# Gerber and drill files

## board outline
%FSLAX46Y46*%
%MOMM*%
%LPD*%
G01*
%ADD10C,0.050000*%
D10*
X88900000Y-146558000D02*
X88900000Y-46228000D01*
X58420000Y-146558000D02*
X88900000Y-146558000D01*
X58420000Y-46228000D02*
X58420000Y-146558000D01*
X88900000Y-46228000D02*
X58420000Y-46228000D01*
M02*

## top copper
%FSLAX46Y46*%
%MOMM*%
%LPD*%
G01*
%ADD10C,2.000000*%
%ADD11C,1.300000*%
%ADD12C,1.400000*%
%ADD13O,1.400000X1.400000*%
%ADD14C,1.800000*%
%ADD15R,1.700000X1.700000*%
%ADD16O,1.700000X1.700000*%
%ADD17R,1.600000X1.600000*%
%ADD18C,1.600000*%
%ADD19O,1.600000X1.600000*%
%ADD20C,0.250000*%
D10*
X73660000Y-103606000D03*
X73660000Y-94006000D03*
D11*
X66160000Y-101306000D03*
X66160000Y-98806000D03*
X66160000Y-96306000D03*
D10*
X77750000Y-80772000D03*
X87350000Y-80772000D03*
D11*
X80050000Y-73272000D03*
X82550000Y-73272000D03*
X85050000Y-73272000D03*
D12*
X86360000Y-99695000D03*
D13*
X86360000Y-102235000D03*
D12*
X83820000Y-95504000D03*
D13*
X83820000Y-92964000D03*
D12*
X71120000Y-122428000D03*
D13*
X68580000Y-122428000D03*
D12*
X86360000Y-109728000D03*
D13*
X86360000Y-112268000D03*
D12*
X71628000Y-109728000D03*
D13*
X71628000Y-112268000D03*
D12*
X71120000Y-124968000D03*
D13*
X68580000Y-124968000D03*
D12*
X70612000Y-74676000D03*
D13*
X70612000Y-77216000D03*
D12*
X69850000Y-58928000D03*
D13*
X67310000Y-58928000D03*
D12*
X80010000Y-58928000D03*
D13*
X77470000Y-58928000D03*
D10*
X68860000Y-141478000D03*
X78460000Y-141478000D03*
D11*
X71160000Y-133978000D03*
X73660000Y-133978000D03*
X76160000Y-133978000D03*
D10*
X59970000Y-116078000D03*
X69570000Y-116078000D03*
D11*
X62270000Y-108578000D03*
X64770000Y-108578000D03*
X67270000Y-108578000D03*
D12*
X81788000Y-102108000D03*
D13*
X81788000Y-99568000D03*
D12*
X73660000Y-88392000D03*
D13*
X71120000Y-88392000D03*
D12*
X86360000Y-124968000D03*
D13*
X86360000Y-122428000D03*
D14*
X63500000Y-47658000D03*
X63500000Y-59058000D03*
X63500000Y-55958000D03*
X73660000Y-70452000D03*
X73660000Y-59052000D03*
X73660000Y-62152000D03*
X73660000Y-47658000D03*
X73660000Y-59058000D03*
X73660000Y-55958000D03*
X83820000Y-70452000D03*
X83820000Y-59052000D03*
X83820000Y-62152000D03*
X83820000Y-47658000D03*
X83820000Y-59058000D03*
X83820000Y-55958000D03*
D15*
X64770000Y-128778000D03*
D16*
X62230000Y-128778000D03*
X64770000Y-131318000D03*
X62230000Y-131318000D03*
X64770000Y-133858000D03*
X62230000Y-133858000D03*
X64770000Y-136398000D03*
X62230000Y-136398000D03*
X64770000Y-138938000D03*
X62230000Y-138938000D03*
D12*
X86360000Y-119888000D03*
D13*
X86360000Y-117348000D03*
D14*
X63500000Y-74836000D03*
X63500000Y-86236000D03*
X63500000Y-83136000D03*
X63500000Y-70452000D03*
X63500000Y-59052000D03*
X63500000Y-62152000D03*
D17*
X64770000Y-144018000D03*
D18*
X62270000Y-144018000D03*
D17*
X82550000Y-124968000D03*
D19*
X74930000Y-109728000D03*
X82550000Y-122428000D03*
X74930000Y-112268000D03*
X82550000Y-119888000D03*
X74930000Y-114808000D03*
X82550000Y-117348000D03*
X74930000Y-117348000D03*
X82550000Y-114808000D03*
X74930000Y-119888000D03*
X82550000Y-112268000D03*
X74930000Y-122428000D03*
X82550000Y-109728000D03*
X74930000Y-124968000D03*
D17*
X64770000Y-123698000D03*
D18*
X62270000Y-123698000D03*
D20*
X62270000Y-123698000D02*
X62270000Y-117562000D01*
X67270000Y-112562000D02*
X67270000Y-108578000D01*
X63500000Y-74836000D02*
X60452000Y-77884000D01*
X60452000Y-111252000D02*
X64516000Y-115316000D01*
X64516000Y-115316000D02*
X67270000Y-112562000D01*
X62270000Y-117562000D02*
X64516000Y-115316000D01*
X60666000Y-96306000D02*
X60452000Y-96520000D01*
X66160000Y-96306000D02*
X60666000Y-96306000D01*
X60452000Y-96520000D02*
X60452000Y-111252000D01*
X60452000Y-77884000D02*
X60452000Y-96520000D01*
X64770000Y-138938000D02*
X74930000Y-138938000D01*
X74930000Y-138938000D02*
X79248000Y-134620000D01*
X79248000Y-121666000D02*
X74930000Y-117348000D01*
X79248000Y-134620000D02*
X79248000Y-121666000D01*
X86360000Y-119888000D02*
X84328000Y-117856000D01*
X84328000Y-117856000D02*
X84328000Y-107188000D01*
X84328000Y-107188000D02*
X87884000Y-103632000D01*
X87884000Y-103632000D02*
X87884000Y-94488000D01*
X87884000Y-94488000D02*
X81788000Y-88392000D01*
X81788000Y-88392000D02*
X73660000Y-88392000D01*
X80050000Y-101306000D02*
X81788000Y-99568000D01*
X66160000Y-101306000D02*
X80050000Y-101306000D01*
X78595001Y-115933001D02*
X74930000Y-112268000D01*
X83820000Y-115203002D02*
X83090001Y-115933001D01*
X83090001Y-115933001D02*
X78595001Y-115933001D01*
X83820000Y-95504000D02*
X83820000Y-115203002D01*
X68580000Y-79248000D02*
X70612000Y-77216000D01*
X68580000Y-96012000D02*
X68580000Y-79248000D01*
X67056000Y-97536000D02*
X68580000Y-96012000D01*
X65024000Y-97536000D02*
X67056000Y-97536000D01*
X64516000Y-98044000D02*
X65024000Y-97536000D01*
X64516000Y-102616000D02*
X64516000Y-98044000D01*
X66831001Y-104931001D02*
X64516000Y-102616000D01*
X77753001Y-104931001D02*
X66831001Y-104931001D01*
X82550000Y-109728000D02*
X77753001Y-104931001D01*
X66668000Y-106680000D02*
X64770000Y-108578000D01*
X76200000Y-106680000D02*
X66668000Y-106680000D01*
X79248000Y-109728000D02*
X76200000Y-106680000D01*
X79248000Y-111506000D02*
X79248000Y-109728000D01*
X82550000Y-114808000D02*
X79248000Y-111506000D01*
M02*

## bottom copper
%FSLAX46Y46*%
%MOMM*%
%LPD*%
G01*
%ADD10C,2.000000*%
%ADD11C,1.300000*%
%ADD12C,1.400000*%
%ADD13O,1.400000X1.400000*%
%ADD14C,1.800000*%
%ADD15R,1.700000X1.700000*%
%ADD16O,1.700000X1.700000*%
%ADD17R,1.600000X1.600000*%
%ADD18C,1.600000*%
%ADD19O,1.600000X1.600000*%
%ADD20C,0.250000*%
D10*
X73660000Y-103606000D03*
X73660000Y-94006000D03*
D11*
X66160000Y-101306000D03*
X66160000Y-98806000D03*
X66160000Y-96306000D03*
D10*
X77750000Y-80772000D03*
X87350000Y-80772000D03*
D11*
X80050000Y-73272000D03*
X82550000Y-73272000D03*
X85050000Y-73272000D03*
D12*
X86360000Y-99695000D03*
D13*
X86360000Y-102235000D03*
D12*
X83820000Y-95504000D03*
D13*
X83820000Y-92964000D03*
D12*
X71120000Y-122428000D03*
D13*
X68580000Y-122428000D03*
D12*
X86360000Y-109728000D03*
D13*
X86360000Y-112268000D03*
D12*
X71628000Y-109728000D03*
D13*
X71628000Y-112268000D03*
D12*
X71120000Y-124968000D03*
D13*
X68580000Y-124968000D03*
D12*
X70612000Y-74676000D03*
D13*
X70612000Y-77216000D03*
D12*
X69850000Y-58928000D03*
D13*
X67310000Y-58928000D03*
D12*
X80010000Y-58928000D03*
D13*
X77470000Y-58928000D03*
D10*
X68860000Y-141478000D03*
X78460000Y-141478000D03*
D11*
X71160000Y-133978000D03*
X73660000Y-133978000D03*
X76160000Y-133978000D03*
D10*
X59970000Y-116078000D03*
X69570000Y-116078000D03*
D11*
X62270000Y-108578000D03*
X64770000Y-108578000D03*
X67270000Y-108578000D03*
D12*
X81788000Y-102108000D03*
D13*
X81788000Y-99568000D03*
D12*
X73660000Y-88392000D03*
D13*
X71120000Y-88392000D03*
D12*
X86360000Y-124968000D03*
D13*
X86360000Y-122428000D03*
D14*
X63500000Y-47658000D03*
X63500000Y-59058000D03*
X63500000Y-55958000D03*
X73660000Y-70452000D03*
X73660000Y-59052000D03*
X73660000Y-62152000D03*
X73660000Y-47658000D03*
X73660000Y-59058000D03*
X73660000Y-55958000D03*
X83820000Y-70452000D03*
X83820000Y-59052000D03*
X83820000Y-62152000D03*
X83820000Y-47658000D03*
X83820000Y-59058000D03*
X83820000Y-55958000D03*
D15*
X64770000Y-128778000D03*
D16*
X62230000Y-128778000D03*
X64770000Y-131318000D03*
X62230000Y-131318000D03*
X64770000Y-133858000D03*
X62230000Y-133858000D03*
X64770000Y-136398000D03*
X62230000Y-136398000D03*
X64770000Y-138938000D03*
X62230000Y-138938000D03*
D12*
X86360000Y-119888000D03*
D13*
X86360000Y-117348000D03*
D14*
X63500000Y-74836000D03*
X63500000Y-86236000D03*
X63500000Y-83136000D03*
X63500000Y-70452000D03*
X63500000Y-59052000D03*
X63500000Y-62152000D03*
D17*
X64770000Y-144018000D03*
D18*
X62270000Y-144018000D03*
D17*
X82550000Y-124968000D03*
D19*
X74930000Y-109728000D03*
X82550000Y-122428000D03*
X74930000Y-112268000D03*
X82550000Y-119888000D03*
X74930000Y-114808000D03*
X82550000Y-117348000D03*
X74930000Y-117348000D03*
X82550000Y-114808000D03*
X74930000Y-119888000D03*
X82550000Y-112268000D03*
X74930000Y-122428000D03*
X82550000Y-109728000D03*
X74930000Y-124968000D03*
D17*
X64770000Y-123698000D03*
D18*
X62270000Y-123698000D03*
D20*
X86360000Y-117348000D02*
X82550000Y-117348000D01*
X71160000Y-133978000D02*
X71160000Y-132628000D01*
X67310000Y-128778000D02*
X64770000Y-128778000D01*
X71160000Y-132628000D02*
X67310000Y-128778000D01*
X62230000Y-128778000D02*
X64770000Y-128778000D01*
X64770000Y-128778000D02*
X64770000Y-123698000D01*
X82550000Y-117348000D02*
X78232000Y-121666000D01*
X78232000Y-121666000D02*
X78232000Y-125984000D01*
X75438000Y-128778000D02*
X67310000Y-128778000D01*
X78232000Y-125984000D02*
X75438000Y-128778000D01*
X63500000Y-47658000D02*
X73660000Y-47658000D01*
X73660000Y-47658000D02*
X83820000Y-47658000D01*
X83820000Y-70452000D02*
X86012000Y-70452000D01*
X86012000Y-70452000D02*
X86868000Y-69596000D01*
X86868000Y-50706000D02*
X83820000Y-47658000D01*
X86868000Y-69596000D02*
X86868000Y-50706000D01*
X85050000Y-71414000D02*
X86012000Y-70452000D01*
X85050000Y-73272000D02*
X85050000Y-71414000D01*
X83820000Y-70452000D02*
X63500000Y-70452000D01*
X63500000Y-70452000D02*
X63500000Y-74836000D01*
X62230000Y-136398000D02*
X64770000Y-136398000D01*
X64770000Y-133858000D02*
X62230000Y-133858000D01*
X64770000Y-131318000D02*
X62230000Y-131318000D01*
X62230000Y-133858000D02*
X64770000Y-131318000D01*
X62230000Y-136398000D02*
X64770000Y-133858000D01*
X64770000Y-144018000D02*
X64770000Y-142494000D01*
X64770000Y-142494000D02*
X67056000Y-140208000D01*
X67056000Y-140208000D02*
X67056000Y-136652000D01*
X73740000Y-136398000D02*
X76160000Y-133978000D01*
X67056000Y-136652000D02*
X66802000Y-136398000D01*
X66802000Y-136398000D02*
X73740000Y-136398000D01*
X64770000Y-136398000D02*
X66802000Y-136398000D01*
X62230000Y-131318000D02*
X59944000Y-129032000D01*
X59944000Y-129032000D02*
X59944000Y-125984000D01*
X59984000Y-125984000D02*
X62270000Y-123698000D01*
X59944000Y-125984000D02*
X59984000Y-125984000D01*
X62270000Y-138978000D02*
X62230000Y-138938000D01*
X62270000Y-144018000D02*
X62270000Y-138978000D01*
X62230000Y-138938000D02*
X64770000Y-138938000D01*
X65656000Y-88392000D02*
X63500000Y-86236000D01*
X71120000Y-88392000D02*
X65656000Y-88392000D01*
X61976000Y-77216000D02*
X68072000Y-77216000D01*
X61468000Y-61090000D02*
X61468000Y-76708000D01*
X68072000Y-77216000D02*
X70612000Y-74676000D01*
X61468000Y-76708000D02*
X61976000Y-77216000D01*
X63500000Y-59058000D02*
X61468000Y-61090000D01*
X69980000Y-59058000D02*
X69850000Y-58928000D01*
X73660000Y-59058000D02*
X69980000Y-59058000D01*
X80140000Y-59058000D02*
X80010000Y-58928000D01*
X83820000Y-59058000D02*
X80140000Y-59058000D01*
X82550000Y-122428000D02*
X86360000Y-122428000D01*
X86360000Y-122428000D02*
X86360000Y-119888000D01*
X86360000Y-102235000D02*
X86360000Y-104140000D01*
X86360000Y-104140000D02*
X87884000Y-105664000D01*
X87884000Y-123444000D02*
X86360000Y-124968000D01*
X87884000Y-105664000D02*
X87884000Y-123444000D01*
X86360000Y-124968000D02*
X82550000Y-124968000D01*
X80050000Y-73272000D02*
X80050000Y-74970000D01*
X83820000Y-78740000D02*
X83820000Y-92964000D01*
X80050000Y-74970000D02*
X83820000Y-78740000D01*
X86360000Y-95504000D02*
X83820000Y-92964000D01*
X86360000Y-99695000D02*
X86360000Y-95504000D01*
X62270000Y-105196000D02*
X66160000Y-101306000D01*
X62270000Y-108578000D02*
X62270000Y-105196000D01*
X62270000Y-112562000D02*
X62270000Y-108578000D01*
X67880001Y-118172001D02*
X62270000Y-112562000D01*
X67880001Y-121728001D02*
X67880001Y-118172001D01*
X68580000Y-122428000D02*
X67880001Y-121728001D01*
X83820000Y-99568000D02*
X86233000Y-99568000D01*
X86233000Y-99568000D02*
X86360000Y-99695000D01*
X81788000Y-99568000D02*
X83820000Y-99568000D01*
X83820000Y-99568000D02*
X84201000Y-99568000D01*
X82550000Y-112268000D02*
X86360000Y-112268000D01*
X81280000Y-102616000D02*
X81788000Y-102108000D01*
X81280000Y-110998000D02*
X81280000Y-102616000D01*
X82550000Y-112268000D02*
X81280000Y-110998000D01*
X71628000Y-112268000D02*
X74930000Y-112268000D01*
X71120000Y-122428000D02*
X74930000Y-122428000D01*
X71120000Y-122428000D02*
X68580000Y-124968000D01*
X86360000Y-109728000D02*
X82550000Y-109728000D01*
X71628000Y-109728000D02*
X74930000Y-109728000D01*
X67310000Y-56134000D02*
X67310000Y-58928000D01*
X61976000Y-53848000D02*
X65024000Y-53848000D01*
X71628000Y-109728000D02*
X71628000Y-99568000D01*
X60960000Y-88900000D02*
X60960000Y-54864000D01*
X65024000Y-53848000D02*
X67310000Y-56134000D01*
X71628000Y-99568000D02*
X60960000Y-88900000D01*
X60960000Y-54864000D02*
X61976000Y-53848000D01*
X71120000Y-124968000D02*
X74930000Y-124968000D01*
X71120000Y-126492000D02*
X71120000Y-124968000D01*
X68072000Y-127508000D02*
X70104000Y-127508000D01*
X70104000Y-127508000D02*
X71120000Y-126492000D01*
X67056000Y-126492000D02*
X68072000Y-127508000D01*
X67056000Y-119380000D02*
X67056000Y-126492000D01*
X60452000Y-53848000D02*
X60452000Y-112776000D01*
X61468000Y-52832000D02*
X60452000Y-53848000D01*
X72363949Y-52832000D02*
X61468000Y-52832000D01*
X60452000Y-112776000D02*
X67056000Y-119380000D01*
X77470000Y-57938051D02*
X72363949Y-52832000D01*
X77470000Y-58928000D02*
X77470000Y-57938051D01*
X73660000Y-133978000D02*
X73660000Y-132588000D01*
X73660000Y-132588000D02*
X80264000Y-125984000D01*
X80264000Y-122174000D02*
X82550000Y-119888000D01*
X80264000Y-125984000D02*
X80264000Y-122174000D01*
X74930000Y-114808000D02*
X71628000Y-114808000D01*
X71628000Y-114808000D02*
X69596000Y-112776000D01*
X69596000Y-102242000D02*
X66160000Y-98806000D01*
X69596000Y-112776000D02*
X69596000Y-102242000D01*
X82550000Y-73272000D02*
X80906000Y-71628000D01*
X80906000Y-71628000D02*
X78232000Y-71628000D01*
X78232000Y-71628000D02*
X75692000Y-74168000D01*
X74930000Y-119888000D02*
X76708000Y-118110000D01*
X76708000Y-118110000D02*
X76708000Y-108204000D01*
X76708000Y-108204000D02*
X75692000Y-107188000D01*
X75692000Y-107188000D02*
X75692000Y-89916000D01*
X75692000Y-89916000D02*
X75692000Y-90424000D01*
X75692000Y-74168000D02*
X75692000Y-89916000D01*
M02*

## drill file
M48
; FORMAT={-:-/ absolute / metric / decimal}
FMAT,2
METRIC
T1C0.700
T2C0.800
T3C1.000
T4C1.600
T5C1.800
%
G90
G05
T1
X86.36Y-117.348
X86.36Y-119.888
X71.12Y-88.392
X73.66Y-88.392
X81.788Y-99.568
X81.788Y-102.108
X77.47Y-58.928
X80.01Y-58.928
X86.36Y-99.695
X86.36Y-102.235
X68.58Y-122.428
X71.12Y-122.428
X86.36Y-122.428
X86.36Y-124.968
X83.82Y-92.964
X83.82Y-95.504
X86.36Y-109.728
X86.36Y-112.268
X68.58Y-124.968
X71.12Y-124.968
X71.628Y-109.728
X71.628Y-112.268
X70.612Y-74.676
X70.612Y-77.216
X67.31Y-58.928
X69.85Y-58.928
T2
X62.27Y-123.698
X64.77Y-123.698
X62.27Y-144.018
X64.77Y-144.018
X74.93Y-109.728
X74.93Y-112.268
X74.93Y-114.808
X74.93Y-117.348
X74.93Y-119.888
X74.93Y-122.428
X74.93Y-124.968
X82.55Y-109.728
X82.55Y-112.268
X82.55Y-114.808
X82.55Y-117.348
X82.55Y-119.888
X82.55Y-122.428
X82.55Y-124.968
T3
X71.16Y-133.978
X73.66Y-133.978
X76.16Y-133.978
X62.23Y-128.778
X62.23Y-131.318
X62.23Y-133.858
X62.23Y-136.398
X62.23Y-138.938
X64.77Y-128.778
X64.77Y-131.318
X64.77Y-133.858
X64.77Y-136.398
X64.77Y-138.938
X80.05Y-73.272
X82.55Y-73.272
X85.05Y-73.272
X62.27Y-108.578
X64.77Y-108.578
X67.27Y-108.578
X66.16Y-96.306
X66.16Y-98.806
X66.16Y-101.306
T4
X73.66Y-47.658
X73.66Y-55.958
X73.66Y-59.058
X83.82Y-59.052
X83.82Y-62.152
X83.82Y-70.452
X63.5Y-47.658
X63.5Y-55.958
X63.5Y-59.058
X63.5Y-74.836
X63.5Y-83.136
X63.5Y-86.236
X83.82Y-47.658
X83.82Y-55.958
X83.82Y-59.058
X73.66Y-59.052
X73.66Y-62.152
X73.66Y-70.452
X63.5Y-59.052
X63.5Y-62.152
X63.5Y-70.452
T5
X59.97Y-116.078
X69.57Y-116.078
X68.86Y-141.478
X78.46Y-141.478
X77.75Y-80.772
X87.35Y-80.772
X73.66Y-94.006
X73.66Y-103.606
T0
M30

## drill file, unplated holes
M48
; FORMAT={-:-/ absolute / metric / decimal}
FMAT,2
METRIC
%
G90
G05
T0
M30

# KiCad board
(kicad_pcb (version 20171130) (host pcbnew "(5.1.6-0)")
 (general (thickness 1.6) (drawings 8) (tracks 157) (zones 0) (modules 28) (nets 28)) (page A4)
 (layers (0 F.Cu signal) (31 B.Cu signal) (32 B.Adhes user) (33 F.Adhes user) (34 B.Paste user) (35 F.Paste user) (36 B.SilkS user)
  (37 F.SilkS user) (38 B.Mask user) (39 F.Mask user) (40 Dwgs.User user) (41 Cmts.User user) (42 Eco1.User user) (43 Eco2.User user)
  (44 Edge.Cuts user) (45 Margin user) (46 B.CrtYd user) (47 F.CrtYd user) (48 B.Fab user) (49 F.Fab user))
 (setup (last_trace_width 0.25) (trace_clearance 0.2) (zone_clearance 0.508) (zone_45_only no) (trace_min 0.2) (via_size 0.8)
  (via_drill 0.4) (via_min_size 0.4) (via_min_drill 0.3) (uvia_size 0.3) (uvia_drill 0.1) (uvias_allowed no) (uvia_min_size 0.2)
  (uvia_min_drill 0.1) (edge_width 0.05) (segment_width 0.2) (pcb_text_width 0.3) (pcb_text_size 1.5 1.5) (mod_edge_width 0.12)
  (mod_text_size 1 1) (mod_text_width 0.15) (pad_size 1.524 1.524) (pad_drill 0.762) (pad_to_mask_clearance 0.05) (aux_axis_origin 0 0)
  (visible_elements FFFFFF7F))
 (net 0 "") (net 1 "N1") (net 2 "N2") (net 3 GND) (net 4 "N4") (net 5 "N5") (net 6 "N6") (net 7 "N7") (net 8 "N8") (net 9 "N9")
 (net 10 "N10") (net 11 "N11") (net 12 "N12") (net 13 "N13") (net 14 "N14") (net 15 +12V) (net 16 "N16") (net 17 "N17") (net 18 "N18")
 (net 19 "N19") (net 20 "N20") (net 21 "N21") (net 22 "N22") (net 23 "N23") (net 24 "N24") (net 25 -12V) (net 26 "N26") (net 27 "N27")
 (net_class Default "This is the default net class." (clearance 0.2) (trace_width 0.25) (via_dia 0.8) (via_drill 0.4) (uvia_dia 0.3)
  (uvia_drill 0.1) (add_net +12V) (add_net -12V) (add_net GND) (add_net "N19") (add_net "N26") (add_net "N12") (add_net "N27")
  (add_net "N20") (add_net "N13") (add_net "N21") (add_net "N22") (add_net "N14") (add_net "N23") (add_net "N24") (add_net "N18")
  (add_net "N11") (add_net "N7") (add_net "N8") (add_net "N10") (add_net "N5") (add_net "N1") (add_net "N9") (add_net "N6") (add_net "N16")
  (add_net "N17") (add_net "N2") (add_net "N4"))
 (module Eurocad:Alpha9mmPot (layer F.Cu) (at 73.66 98.806 270)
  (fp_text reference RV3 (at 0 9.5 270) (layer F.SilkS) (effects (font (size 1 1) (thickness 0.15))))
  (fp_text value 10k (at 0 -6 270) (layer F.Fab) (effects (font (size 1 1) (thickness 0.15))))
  (pad "" thru_hole circle (at 4.8 0 270) (size 2 2) (drill 1.8) (layers *.Cu *.Mask F.SilkS))
  (pad "" thru_hole circle (at -4.8 0 270) (size 2 2) (drill 1.8) (layers *.Cu *.Mask F.SilkS))
  (pad 3 thru_hole circle (at 2.5 7.5 270) (size 1.3 1.3) (drill 1) (layers *.Cu *.Mask F.SilkS) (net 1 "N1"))
  (pad 2 thru_hole circle (at 0 7.5 270) (size 1.3 1.3) (drill 1) (layers *.Cu *.Mask F.SilkS) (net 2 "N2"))
  (pad 1 thru_hole circle (at -2.5 7.5 270) (size 1.3 1.3) (drill 1) (layers *.Cu *.Mask F.SilkS) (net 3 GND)))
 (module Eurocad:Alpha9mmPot (layer F.Cu) (at 82.55 80.772 180)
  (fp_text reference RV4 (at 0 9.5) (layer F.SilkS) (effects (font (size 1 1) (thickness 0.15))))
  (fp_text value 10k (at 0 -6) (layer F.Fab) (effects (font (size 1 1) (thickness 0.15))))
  (pad "" thru_hole circle (at 4.8 0 180) (size 2 2) (drill 1.8) (layers *.Cu *.Mask F.SilkS))
  (pad "" thru_hole circle (at -4.8 0 180) (size 2 2) (drill 1.8) (layers *.Cu *.Mask F.SilkS))
  (pad 3 thru_hole circle (at 2.5 7.5 180) (size 1.3 1.3) (drill 1) (layers *.Cu *.Mask F.SilkS) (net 1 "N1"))
  (pad 2 thru_hole circle (at 0 7.5 180) (size 1.3 1.3) (drill 1) (layers *.Cu *.Mask F.SilkS) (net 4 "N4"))
  (pad 1 thru_hole circle (at -2.5 7.5 180) (size 1.3 1.3) (drill 1) (layers *.Cu *.Mask F.SilkS) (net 3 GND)))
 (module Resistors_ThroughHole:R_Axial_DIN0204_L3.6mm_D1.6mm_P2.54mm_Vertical (layer F.Cu) (at 86.36 99.695 270)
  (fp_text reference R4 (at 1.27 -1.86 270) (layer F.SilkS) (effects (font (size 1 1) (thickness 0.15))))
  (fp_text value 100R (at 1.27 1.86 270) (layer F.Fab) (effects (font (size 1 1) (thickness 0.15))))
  (pad 1 thru_hole circle (at 0 0 270) (size 1.4 1.4) (drill 0.7) (layers *.Cu *.Mask) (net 1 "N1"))
  (pad 2 thru_hole oval (at 2.54 0 270) (size 1.4 1.4) (drill 0.7) (layers *.Cu *.Mask) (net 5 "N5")))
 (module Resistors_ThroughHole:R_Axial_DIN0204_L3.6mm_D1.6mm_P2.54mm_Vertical (layer F.Cu) (at 83.82 95.504 90)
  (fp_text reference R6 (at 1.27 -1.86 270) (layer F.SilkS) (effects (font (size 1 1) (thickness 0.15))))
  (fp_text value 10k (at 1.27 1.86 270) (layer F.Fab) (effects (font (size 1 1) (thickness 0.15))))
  (pad 1 thru_hole circle (at 0 0 90) (size 1.4 1.4) (drill 0.7) (layers *.Cu *.Mask) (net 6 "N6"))
  (pad 2 thru_hole oval (at 2.54 0 90) (size 1.4 1.4) (drill 0.7) (layers *.Cu *.Mask) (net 1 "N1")))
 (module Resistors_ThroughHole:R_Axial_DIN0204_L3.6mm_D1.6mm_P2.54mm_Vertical (layer F.Cu) (at 71.12 122.428 180)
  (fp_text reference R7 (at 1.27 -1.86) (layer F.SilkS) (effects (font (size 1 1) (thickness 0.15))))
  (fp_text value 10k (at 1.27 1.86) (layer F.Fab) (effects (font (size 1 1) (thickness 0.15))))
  (pad 1 thru_hole circle (at 0 0 180) (size 1.4 1.4) (drill 0.7) (layers *.Cu *.Mask) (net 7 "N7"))
  (pad 2 thru_hole oval (at 2.54 0 180) (size 1.4 1.4) (drill 0.7) (layers *.Cu *.Mask) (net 1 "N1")))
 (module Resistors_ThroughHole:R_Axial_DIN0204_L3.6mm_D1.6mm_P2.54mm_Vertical (layer F.Cu) (at 86.36 109.728 270)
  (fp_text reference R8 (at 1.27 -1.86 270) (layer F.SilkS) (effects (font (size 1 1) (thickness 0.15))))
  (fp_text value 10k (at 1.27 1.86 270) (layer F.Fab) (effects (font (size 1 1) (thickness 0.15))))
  (pad 1 thru_hole circle (at 0 0 270) (size 1.4 1.4) (drill 0.7) (layers *.Cu *.Mask) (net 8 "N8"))
  (pad 2 thru_hole oval (at 2.54 0 270) (size 1.4 1.4) (drill 0.7) (layers *.Cu *.Mask) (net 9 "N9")))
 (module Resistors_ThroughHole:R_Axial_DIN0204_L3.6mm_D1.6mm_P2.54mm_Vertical (layer F.Cu) (at 71.628 109.728 270)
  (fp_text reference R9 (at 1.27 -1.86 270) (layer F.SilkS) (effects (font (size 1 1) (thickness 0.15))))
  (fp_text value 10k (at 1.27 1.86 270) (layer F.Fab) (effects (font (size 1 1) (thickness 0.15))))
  (pad 1 thru_hole circle (at 0 0 270) (size 1.4 1.4) (drill 0.7) (layers *.Cu *.Mask) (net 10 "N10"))
  (pad 2 thru_hole oval (at 2.54 0 270) (size 1.4 1.4) (drill 0.7) (layers *.Cu *.Mask) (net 6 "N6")))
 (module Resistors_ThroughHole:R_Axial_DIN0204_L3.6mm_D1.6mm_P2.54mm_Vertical (layer F.Cu) (at 71.12 124.968 180)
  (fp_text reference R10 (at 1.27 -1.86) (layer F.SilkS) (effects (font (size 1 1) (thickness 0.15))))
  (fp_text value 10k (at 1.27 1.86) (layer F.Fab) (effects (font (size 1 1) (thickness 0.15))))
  (pad 1 thru_hole circle (at 0 0 180) (size 1.4 1.4) (drill 0.7) (layers *.Cu *.Mask) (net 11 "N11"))
  (pad 2 thru_hole oval (at 2.54 0 180) (size 1.4 1.4) (drill 0.7) (layers *.Cu *.Mask) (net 7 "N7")))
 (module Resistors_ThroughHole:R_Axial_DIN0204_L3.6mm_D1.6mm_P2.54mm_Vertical (layer F.Cu) (at 70.612 74.676 270)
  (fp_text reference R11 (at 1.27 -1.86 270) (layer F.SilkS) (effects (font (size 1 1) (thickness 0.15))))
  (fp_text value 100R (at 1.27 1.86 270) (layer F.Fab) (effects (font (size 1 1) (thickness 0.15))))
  (pad 1 thru_hole circle (at 0 0 270) (size 1.4 1.4) (drill 0.7) (layers *.Cu *.Mask) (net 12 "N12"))
  (pad 2 thru_hole oval (at 2.54 0 270) (size 1.4 1.4) (drill 0.7) (layers *.Cu *.Mask) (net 8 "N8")))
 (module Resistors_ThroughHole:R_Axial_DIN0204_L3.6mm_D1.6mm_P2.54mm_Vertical (layer F.Cu) (at 69.85 58.928 180)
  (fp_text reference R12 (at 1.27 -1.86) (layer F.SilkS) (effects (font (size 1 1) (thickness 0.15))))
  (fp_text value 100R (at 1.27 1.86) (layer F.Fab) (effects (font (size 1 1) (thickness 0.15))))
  (pad 1 thru_hole circle (at 0 0 180) (size 1.4 1.4) (drill 0.7) (layers *.Cu *.Mask) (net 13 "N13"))
  (pad 2 thru_hole oval (at 2.54 0 180) (size 1.4 1.4) (drill 0.7) (layers *.Cu *.Mask) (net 10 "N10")))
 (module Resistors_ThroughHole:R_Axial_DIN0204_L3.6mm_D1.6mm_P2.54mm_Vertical (layer F.Cu) (at 80.01 58.928 180)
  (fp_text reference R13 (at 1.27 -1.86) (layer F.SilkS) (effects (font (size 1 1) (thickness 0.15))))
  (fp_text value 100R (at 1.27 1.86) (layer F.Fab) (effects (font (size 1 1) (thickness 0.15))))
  (pad 1 thru_hole circle (at 0 0 180) (size 1.4 1.4) (drill 0.7) (layers *.Cu *.Mask) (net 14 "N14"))
  (pad 2 thru_hole oval (at 2.54 0 180) (size 1.4 1.4) (drill 0.7) (layers *.Cu *.Mask) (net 11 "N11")))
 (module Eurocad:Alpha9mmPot (layer F.Cu) (at 73.66 141.478 180)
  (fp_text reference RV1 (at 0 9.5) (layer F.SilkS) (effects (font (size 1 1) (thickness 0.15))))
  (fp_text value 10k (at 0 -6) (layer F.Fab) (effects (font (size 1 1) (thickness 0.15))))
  (pad "" thru_hole circle (at 4.8 0 180) (size 2 2) (drill 1.8) (layers *.Cu *.Mask F.SilkS))
  (pad "" thru_hole circle (at -4.8 0 180) (size 2 2) (drill 1.8) (layers *.Cu *.Mask F.SilkS))
  (pad 3 thru_hole circle (at 2.5 7.5 180) (size 1.3 1.3) (drill 1) (layers *.Cu *.Mask F.SilkS) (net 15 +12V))
  (pad 2 thru_hole circle (at 0 7.5 180) (size 1.3 1.3) (drill 1) (layers *.Cu *.Mask F.SilkS) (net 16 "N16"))
  (pad 1 thru_hole circle (at -2.5 7.5 180) (size 1.3 1.3) (drill 1) (layers *.Cu *.Mask F.SilkS) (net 3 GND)))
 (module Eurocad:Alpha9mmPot (layer F.Cu) (at 64.77 116.078 180)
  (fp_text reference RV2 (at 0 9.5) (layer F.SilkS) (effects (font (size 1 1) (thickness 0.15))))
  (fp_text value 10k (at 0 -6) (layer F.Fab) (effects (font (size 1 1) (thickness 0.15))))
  (pad "" thru_hole circle (at 4.8 0 180) (size 2 2) (drill 1.8) (layers *.Cu *.Mask F.SilkS))
  (pad "" thru_hole circle (at -4.8 0 180) (size 2 2) (drill 1.8) (layers *.Cu *.Mask F.SilkS))
  (pad 3 thru_hole circle (at 2.5 7.5 180) (size 1.3 1.3) (drill 1) (layers *.Cu *.Mask F.SilkS) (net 1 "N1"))
  (pad 2 thru_hole circle (at 0 7.5 180) (size 1.3 1.3) (drill 1) (layers *.Cu *.Mask F.SilkS) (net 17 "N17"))
  (pad 1 thru_hole circle (at -2.5 7.5 180) (size 1.3 1.3) (drill 1) (layers *.Cu *.Mask F.SilkS) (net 3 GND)))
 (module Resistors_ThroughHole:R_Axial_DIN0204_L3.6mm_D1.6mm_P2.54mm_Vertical (layer F.Cu) (at 81.788 102.108 90)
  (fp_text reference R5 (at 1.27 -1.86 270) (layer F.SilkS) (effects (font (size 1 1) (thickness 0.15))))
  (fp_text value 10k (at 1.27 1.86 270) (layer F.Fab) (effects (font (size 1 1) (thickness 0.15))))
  (pad 1 thru_hole circle (at 0 0 90) (size 1.4 1.4) (drill 0.7) (layers *.Cu *.Mask) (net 9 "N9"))
  (pad 2 thru_hole oval (at 2.54 0 90) (size 1.4 1.4) (drill 0.7) (layers *.Cu *.Mask) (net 1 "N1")))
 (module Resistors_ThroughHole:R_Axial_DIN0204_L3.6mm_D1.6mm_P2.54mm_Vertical (layer F.Cu) (at 73.66 88.392 180)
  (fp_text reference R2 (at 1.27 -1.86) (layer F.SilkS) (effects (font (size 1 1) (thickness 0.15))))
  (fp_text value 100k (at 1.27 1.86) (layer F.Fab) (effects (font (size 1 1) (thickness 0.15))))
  (pad 1 thru_hole circle (at 0 0 180) (size 1.4 1.4) (drill 0.7) (layers *.Cu *.Mask) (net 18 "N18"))
  (pad 2 thru_hole oval (at 2.54 0 180) (size 1.4 1.4) (drill 0.7) (layers *.Cu *.Mask) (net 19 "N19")))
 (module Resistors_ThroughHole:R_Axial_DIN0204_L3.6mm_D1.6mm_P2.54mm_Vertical (layer F.Cu) (at 86.36 124.968 90)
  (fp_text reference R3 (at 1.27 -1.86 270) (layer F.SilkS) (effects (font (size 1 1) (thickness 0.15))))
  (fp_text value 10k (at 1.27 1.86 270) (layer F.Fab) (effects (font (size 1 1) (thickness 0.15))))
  (pad 1 thru_hole circle (at 0 0 90) (size 1.4 1.4) (drill 0.7) (layers *.Cu *.Mask) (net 5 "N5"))
  (pad 2 thru_hole oval (at 2.54 0 90) (size 1.4 1.4) (drill 0.7) (layers *.Cu *.Mask) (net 18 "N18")))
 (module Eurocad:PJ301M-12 (layer F.Cu) (at 63.5 52.578)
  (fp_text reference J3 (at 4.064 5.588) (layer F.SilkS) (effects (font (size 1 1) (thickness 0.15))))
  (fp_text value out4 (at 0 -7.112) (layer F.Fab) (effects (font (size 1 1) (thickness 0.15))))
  (pad 3 thru_hole circle (at 0 -4.92) (size 1.8 1.8) (drill 1.6) (layers *.Cu *.Mask F.SilkS) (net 3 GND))
  (pad 1 thru_hole circle (at 0 6.48) (size 1.8 1.8) (drill 1.6) (layers *.Cu *.Mask F.SilkS) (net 12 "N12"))
  (pad 2 thru_hole circle (at 0 3.38) (size 1.8 1.8) (drill 1.6) (layers *.Cu *.Mask F.SilkS) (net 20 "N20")))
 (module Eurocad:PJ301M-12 (layer F.Cu) (at 73.66 65.532 180)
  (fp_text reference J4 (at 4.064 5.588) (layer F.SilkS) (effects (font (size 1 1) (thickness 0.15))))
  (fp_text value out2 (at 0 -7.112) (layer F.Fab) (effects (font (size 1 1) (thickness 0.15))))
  (pad 3 thru_hole circle (at 0 -4.92 180) (size 1.8 1.8) (drill 1.6) (layers *.Cu *.Mask F.SilkS) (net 3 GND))
  (pad 1 thru_hole circle (at 0 6.48 180) (size 1.8 1.8) (drill 1.6) (layers *.Cu *.Mask F.SilkS) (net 13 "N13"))
  (pad 2 thru_hole circle (at 0 3.38 180) (size 1.8 1.8) (drill 1.6) (layers *.Cu *.Mask F.SilkS) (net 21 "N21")))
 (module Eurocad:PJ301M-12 (layer F.Cu) (at 73.66 52.578)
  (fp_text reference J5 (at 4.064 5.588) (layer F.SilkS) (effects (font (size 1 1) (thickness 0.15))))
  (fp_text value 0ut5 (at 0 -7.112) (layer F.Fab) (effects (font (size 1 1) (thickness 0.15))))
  (pad 3 thru_hole circle (at 0 -4.92) (size 1.8 1.8) (drill 1.6) (layers *.Cu *.Mask F.SilkS) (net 3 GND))
  (pad 1 thru_hole circle (at 0 6.48) (size 1.8 1.8) (drill 1.6) (layers *.Cu *.Mask F.SilkS) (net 13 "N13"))
  (pad 2 thru_hole circle (at 0 3.38) (size 1.8 1.8) (drill 1.6) (layers *.Cu *.Mask F.SilkS) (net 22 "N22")))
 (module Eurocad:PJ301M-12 (layer F.Cu) (at 83.82 65.532 180)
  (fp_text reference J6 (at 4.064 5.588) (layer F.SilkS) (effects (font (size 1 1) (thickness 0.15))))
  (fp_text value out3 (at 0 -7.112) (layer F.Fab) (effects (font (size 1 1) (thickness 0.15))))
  (pad 3 thru_hole circle (at 0 -4.92 180) (size 1.8 1.8) (drill 1.6) (layers *.Cu *.Mask F.SilkS) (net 3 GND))
  (pad 1 thru_hole circle (at 0 6.48 180) (size 1.8 1.8) (drill 1.6) (layers *.Cu *.Mask F.SilkS) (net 14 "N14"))
  (pad 2 thru_hole circle (at 0 3.38 180) (size 1.8 1.8) (drill 1.6) (layers *.Cu *.Mask F.SilkS) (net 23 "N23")))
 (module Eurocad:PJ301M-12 (layer F.Cu) (at 83.82 52.578)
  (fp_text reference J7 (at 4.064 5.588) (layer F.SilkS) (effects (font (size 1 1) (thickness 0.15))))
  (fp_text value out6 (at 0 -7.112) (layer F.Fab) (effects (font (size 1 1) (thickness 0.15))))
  (pad 3 thru_hole circle (at 0 -4.92) (size 1.8 1.8) (drill 1.6) (layers *.Cu *.Mask F.SilkS) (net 3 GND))
  (pad 1 thru_hole circle (at 0 6.48) (size 1.8 1.8) (drill 1.6) (layers *.Cu *.Mask F.SilkS) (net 14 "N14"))
  (pad 2 thru_hole circle (at 0 3.38) (size 1.8 1.8) (drill 1.6) (layers *.Cu *.Mask F.SilkS) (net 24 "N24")))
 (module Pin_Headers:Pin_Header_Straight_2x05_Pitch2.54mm (layer B.Cu) (at 64.77 128.778 180)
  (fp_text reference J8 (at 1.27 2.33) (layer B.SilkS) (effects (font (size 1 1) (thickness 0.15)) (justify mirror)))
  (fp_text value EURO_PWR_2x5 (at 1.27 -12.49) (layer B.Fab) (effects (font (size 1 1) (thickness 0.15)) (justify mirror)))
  (pad 1 thru_hole rect (at 0 0 180) (size 1.7 1.7) (drill 1) (layers *.Cu *.Mask) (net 15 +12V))
  (pad 2 thru_hole oval (at 2.54 0 180) (size 1.7 1.7) (drill 1) (layers *.Cu *.Mask) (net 15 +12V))
  (pad 3 thru_hole oval (at 0 -2.54 180) (size 1.7 1.7) (drill 1) (layers *.Cu *.Mask) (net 3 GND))
  (pad 4 thru_hole oval (at 2.54 -2.54 180) (size 1.7 1.7) (drill 1) (layers *.Cu *.Mask) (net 3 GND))
  (pad 5 thru_hole oval (at 0 -5.08 180) (size 1.7 1.7) (drill 1) (layers *.Cu *.Mask) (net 3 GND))
  (pad 6 thru_hole oval (at 2.54 -5.08 180) (size 1.7 1.7) (drill 1) (layers *.Cu *.Mask) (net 3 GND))
  (pad 7 thru_hole oval (at 0 -7.62 180) (size 1.7 1.7) (drill 1) (layers *.Cu *.Mask) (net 3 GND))
  (pad 8 thru_hole oval (at 2.54 -7.62 180) (size 1.7 1.7) (drill 1) (layers *.Cu *.Mask) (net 3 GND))
  (pad 9 thru_hole oval (at 0 -10.16 180) (size 1.7 1.7) (drill 1) (layers *.Cu *.Mask) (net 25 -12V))
  (pad 10 thru_hole oval (at 2.54 -10.16 180) (size 1.7 1.7) (drill 1) (layers *.Cu *.Mask) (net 25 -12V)))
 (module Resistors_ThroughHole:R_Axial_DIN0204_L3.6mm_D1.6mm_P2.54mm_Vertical (layer F.Cu) (at 86.36 119.888 90)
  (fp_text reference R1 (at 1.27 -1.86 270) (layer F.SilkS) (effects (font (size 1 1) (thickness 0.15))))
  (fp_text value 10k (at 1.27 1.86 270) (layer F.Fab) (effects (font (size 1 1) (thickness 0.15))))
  (pad 1 thru_hole circle (at 0 0 90) (size 1.4 1.4) (drill 0.7) (layers *.Cu *.Mask) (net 18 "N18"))
  (pad 2 thru_hole oval (at 2.54 0 90) (size 1.4 1.4) (drill 0.7) (layers *.Cu *.Mask) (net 15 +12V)))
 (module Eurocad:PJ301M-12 (layer F.Cu) (at 63.5 79.756)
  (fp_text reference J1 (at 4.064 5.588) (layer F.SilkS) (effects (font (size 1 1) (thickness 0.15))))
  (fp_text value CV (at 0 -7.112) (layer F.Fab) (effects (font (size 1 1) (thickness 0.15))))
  (pad 3 thru_hole circle (at 0 -4.92) (size 1.8 1.8) (drill 1.6) (layers *.Cu *.Mask F.SilkS) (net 3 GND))
  (pad 1 thru_hole circle (at 0 6.48) (size 1.8 1.8) (drill 1.6) (layers *.Cu *.Mask F.SilkS) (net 19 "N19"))
  (pad 2 thru_hole circle (at 0 3.38) (size 1.8 1.8) (drill 1.6) (layers *.Cu *.Mask F.SilkS) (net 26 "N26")))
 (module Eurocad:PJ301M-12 (layer F.Cu) (at 63.5 65.532 180)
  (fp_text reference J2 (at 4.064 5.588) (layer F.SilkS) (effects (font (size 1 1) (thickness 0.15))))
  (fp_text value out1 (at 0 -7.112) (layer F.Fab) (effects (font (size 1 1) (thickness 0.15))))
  (pad 3 thru_hole circle (at 0 -4.92 180) (size 1.8 1.8) (drill 1.6) (layers *.Cu *.Mask F.SilkS) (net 3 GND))
  (pad 1 thru_hole circle (at 0 6.48 180) (size 1.8 1.8) (drill 1.6) (layers *.Cu *.Mask F.SilkS) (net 12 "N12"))
  (pad 2 thru_hole circle (at 0 3.38 180) (size 1.8 1.8) (drill 1.6) (layers *.Cu *.Mask F.SilkS) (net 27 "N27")))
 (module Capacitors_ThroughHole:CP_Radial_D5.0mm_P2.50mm (layer B.Cu) (at 64.77 144.018 180)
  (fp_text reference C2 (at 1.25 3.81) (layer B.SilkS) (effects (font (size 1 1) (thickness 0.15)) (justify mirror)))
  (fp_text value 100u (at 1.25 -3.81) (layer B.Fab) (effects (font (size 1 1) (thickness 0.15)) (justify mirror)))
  (pad 1 thru_hole rect (at 0 0 180) (size 1.6 1.6) (drill 0.8) (layers *.Cu *.Mask) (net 3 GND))
  (pad 2 thru_hole circle (at 2.5 0 180) (size 1.6 1.6) (drill 0.8) (layers *.Cu *.Mask) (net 25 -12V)))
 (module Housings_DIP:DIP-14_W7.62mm (layer F.Cu) (at 82.55 124.968 180)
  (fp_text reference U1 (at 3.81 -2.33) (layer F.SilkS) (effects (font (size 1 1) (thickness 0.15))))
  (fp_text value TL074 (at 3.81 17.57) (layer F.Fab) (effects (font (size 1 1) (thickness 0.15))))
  (pad 1 thru_hole rect (at 0 0 180) (size 1.6 1.6) (drill 0.8) (layers *.Cu *.Mask) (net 5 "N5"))
  (pad 8 thru_hole oval (at 7.62 15.24 180) (size 1.6 1.6) (drill 0.8) (layers *.Cu *.Mask) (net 10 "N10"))
  (pad 2 thru_hole oval (at 0 2.54 180) (size 1.6 1.6) (drill 0.8) (layers *.Cu *.Mask) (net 18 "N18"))
  (pad 9 thru_hole oval (at 7.62 12.7 180) (size 1.6 1.6) (drill 0.8) (layers *.Cu *.Mask) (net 6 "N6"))
  (pad 3 thru_hole oval (at 0 5.08 180) (size 1.6 1.6) (drill 0.8) (layers *.Cu *.Mask) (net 16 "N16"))
  (pad 10 thru_hole oval (at 7.62 10.16 180) (size 1.6 1.6) (drill 0.8) (layers *.Cu *.Mask) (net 2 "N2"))
  (pad 4 thru_hole oval (at 0 7.62 180) (size 1.6 1.6) (drill 0.8) (layers *.Cu *.Mask) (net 15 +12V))
  (pad 11 thru_hole oval (at 7.62 7.62 180) (size 1.6 1.6) (drill 0.8) (layers *.Cu *.Mask) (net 25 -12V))
  (pad 5 thru_hole oval (at 0 10.16 180) (size 1.6 1.6) (drill 0.8) (layers *.Cu *.Mask) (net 17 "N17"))
  (pad 12 thru_hole oval (at 7.62 5.08 180) (size 1.6 1.6) (drill 0.8) (layers *.Cu *.Mask) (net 4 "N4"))
  (pad 6 thru_hole oval (at 0 12.7 180) (size 1.6 1.6) (drill 0.8) (layers *.Cu *.Mask) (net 9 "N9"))
  (pad 13 thru_hole oval (at 7.62 2.54 180) (size 1.6 1.6) (drill 0.8) (layers *.Cu *.Mask) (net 7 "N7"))
  (pad 7 thru_hole oval (at 0 15.24 180) (size 1.6 1.6) (drill 0.8) (layers *.Cu *.Mask) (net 8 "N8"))
  (pad 14 thru_hole oval (at 7.62 0 180) (size 1.6 1.6) (drill 0.8) (layers *.Cu *.Mask) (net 11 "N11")))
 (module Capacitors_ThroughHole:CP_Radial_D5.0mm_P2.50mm (layer B.Cu) (at 64.77 123.698 180)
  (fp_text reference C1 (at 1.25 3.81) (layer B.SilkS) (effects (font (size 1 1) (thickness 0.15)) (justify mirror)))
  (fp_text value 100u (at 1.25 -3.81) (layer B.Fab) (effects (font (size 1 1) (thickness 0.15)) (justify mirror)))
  (pad 1 thru_hole rect (at 0 0 180) (size 1.6 1.6) (drill 0.8) (layers *.Cu *.Mask) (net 15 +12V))
  (pad 2 thru_hole circle (at 2.5 0 180) (size 1.6 1.6) (drill 0.8) (layers *.Cu *.Mask) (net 3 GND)))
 (gr_line (start 88.9 146.558) (end 88.9 46.228) (layer Edge.Cuts) (width 0.05))
 (gr_line (start 58.42 146.558) (end 88.9 146.558) (layer Edge.Cuts) (width 0.05))
 (gr_line (start 58.42 46.228) (end 58.42 146.558) (layer Edge.Cuts) (width 0.05))
 (gr_line (start 88.9 46.228) (end 58.42 46.228) (layer Edge.Cuts) (width 0.05))
 (segment (start 86.36 117.348) (end 82.55 117.348) (width 0.25) (layer B.Cu) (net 15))
 (segment (start 71.16 133.978) (end 71.16 132.628) (width 0.25) (layer B.Cu) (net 15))
 (segment (start 67.31 128.778) (end 64.77 128.778) (width 0.25) (layer B.Cu) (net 15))
 (segment (start 71.16 132.628) (end 67.31 128.778) (width 0.25) (layer B.Cu) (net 15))
 (segment (start 62.23 128.778) (end 64.77 128.778) (width 0.25) (layer B.Cu) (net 15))
 (segment (start 64.77 128.778) (end 64.77 123.698) (width 0.25) (layer B.Cu) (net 15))
 (segment (start 82.55 117.348) (end 78.232 121.666) (width 0.25) (layer B.Cu) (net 15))
 (segment (start 78.232 121.666) (end 78.232 125.984) (width 0.25) (layer B.Cu) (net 15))
 (segment (start 75.438 128.778) (end 67.31 128.778) (width 0.25) (layer B.Cu) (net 15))
 (segment (start 78.232 125.984) (end 75.438 128.778) (width 0.25) (layer B.Cu) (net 15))
 (segment (start 63.5 47.658) (end 73.66 47.658) (width 0.25) (layer B.Cu) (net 3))
 (segment (start 73.66 47.658) (end 83.82 47.658) (width 0.25) (layer B.Cu) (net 3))
 (segment (start 83.82 70.452) (end 86.012 70.452) (width 0.25) (layer B.Cu) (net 3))
 (segment (start 86.012 70.452) (end 86.868 69.596) (width 0.25) (layer B.Cu) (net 3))
 (segment (start 86.868 50.706) (end 83.82 47.658) (width 0.25) (layer B.Cu) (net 3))
 (segment (start 86.868 69.596) (end 86.868 50.706) (width 0.25) (layer B.Cu) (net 3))
 (segment (start 85.05 71.414) (end 86.012 70.452) (width 0.25) (layer B.Cu) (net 3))
 (segment (start 85.05 73.272) (end 85.05 71.414) (width 0.25) (layer B.Cu) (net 3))
 (segment (start 83.82 70.452) (end 63.5 70.452) (width 0.25) (layer B.Cu) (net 3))
 (segment (start 63.5 70.452) (end 63.5 74.836) (width 0.25) (layer B.Cu) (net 3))
 (segment (start 62.23 136.398) (end 64.77 136.398) (width 0.25) (layer B.Cu) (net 3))
 (segment (start 64.77 133.858) (end 62.23 133.858) (width 0.25) (layer B.Cu) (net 3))
 (segment (start 64.77 131.318) (end 62.23 131.318) (width 0.25) (layer B.Cu) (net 3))
 (segment (start 62.23 133.858) (end 64.77 131.318) (width 0.25) (layer B.Cu) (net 3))
 (segment (start 62.23 136.398) (end 64.77 133.858) (width 0.25) (layer B.Cu) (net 3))
 (segment (start 64.77 144.018) (end 64.77 142.494) (width 0.25) (layer B.Cu) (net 3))
 (segment (start 64.77 142.494) (end 67.056 140.208) (width 0.25) (layer B.Cu) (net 3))
 (segment (start 67.056 140.208) (end 67.056 136.652) (width 0.25) (layer B.Cu) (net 3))
 (segment (start 73.74 136.398) (end 76.16 133.978) (width 0.25) (layer B.Cu) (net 3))
 (segment (start 67.056 136.652) (end 66.802 136.398) (width 0.25) (layer B.Cu) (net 3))
 (segment (start 66.802 136.398) (end 73.74 136.398) (width 0.25) (layer B.Cu) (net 3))
 (segment (start 64.77 136.398) (end 66.802 136.398) (width 0.25) (layer B.Cu) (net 3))
 (segment (start 62.23 131.318) (end 59.944 129.032) (width 0.25) (layer B.Cu) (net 3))
 (segment (start 59.944 129.032) (end 59.944 125.984) (width 0.25) (layer B.Cu) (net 3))
 (segment (start 59.984 125.984) (end 62.27 123.698) (width 0.25) (layer B.Cu) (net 3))
 (segment (start 59.944 125.984) (end 59.984 125.984) (width 0.25) (layer B.Cu) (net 3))
 (segment (start 62.27 123.698) (end 62.27 117.562) (width 0.25) (layer F.Cu) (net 3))
 (segment (start 67.27 112.562) (end 67.27 108.578) (width 0.25) (layer F.Cu) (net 3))
 (segment (start 63.5 74.836) (end 60.452 77.884) (width 0.25) (layer F.Cu) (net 3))
 (segment (start 60.452 111.252) (end 64.516 115.316) (width 0.25) (layer F.Cu) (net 3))
 (segment (start 64.516 115.316) (end 67.27 112.562) (width 0.25) (layer F.Cu) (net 3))
 (segment (start 62.27 117.562) (end 64.516 115.316) (width 0.25) (layer F.Cu) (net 3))
 (segment (start 60.666 96.306) (end 60.452 96.52) (width 0.25) (layer F.Cu) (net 3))
 (segment (start 66.16 96.306) (end 60.666 96.306) (width 0.25) (layer F.Cu) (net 3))
 (segment (start 60.452 96.52) (end 60.452 111.252) (width 0.25) (layer F.Cu) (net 3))
 (segment (start 60.452 77.884) (end 60.452 96.52) (width 0.25) (layer F.Cu) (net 3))
 (segment (start 62.27 138.978) (end 62.23 138.938) (width 0.25) (layer B.Cu) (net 25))
 (segment (start 62.27 144.018) (end 62.27 138.978) (width 0.25) (layer B.Cu) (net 25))
 (segment (start 62.23 138.938) (end 64.77 138.938) (width 0.25) (layer B.Cu) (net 25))
 (segment (start 64.77 138.938) (end 74.93 138.938) (width 0.25) (layer F.Cu) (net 25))
 (segment (start 74.93 138.938) (end 79.248 134.62) (width 0.25) (layer F.Cu) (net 25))
 (segment (start 79.248 121.666) (end 74.93 117.348) (width 0.25) (layer F.Cu) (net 25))
 (segment (start 79.248 134.62) (end 79.248 121.666) (width 0.25) (layer F.Cu) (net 25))
 (segment (start 65.656 88.392) (end 63.5 86.236) (width 0.25) (layer B.Cu) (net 19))
 (segment (start 71.12 88.392) (end 65.656 88.392) (width 0.25) (layer B.Cu) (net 19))
 (segment (start 61.976 77.216) (end 68.072 77.216) (width 0.25) (layer B.Cu) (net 12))
 (segment (start 61.468 61.09) (end 61.468 76.708) (width 0.25) (layer B.Cu) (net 12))
 (segment (start 68.072 77.216) (end 70.612 74.676) (width 0.25) (layer B.Cu) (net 12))
 (segment (start 61.468 76.708) (end 61.976 77.216) (width 0.25) (layer B.Cu) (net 12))
 (segment (start 63.5 59.058) (end 61.468 61.09) (width 0.25) (layer B.Cu) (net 12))
 (segment (start 69.98 59.058) (end 69.85 58.928) (width 0.25) (layer B.Cu) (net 13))
 (segment (start 73.66 59.058) (end 69.98 59.058) (width 0.25) (layer B.Cu) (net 13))
 (segment (start 80.14 59.058) (end 80.01 58.928) (width 0.25) (layer B.Cu) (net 14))
 (segment (start 83.82 59.058) (end 80.14 59.058) (width 0.25) (layer B.Cu) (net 14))
 (segment (start 82.55 122.428) (end 86.36 122.428) (width 0.25) (layer B.Cu) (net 18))
 (segment (start 86.36 122.428) (end 86.36 119.888) (width 0.25) (layer B.Cu) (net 18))
 (segment (start 86.36 119.888) (end 84.328 117.856) (width 0.25) (layer F.Cu) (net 18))
 (segment (start 84.328 117.856) (end 84.328 107.188) (width 0.25) (layer F.Cu) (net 18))
 (segment (start 84.328 107.188) (end 87.884 103.632) (width 0.25) (layer F.Cu) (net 18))
 (segment (start 87.884 103.632) (end 87.884 94.488) (width 0.25) (layer F.Cu) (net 18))
 (segment (start 87.884 94.488) (end 81.788 88.392) (width 0.25) (layer F.Cu) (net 18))
 (segment (start 81.788 88.392) (end 73.66 88.392) (width 0.25) (layer F.Cu) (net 18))
 (segment (start 86.36 102.235) (end 86.36 104.14) (width 0.25) (layer B.Cu) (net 5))
 (segment (start 86.36 104.14) (end 87.884 105.664) (width 0.25) (layer B.Cu) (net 5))
 (segment (start 87.884 123.444) (end 86.36 124.968) (width 0.25) (layer B.Cu) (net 5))
 (segment (start 87.884 105.664) (end 87.884 123.444) (width 0.25) (layer B.Cu) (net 5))
 (segment (start 86.36 124.968) (end 82.55 124.968) (width 0.25) (layer B.Cu) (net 5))
 (segment (start 80.05 73.272) (end 80.05 74.97) (width 0.25) (layer B.Cu) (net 1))
 (segment (start 83.82 78.74) (end 83.82 92.964) (width 0.25) (layer B.Cu) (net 1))
 (segment (start 80.05 74.97) (end 83.82 78.74) (width 0.25) (layer B.Cu) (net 1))
 (segment (start 86.36 95.504) (end 83.82 92.964) (width 0.25) (layer B.Cu) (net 1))
 (segment (start 86.36 99.695) (end 86.36 95.504) (width 0.25) (layer B.Cu) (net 1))
 (segment (start 62.27 105.196) (end 66.16 101.306) (width 0.25) (layer B.Cu) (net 1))
 (segment (start 62.27 108.578) (end 62.27 105.196) (width 0.25) (layer B.Cu) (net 1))
 (segment (start 62.27 112.562) (end 62.27 108.578) (width 0.25) (layer B.Cu) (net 1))
 (segment (start 67.880001 118.172001) (end 62.27 112.562) (width 0.25) (layer B.Cu) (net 1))
 (segment (start 67.880001 121.728001) (end 67.880001 118.172001) (width 0.25) (layer B.Cu) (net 1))
 (segment (start 68.58 122.428) (end 67.880001 121.728001) (width 0.25) (layer B.Cu) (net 1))
 (segment (start 83.82 99.568) (end 86.233 99.568) (width 0.25) (layer B.Cu) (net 1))
 (segment (start 86.233 99.568) (end 86.36 99.695) (width 0.25) (layer B.Cu) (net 1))
 (segment (start 81.788 99.568) (end 83.82 99.568) (width 0.25) (layer B.Cu) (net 1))
 (segment (start 83.82 99.568) (end 84.201 99.568) (width 0.25) (layer B.Cu) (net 1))
 (segment (start 80.05 101.306) (end 81.788 99.568) (width 0.25) (layer F.Cu) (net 1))
 (segment (start 66.16 101.306) (end 80.05 101.306) (width 0.25) (layer F.Cu) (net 1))
 (segment (start 82.55 112.268) (end 86.36 112.268) (width 0.25) (layer B.Cu) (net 9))
 (segment (start 81.28 102.616) (end 81.788 102.108) (width 0.25) (layer B.Cu) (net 9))
 (segment (start 81.28 110.998) (end 81.28 102.616) (width 0.25) (layer B.Cu) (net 9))
 (segment (start 82.55 112.268) (end 81.28 110.998) (width 0.25) (layer B.Cu) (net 9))
 (segment (start 71.628 112.268) (end 74.93 112.268) (width 0.25) (layer B.Cu) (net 6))
 (segment (start 78.595001 115.933001) (end 74.93 112.268) (width 0.25) (layer F.Cu) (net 6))
 (segment (start 83.82 115.203002) (end 83.090001 115.933001) (width 0.25) (layer F.Cu) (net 6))
 (segment (start 83.090001 115.933001) (end 78.595001 115.933001) (width 0.25) (layer F.Cu) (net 6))
 (segment (start 83.82 95.504) (end 83.82 115.203002) (width 0.25) (layer F.Cu) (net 6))
 (segment (start 71.12 122.428) (end 74.93 122.428) (width 0.25) (layer B.Cu) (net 7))
 (segment (start 71.12 122.428) (end 68.58 124.968) (width 0.25) (layer B.Cu) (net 7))
 (segment (start 86.36 109.728) (end 82.55 109.728) (width 0.25) (layer B.Cu) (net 8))
 (segment (start 68.58 79.248) (end 70.612 77.216) (width 0.25) (layer F.Cu) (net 8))
 (segment (start 68.58 96.012) (end 68.58 79.248) (width 0.25) (layer F.Cu) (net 8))
 (segment (start 67.056 97.536) (end 68.58 96.012) (width 0.25) (layer F.Cu) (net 8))
 (segment (start 65.024 97.536) (end 67.056 97.536) (width 0.25) (layer F.Cu) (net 8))
 (segment (start 64.516 98.044) (end 65.024 97.536) (width 0.25) (layer F.Cu) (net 8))
 (segment (start 64.516 102.616) (end 64.516 98.044) (width 0.25) (layer F.Cu) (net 8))
 (segment (start 66.831001 104.931001) (end 64.516 102.616) (width 0.25) (layer F.Cu) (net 8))
 (segment (start 77.753001 104.931001) (end 66.831001 104.931001) (width 0.25) (layer F.Cu) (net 8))
 (segment (start 82.55 109.728) (end 77.753001 104.931001) (width 0.25) (layer F.Cu) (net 8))
 (segment (start 71.628 109.728) (end 74.93 109.728) (width 0.25) (layer B.Cu) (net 10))
 (segment (start 67.31 56.134) (end 67.31 58.928) (width 0.25) (layer B.Cu) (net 10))
 (segment (start 61.976 53.848) (end 65.024 53.848) (width 0.25) (layer B.Cu) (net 10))
 (segment (start 71.628 109.728) (end 71.628 99.568) (width 0.25) (layer B.Cu) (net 10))
 (segment (start 60.96 88.9) (end 60.96 54.864) (width 0.25) (layer B.Cu) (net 10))
 (segment (start 65.024 53.848) (end 67.31 56.134) (width 0.25) (layer B.Cu) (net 10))
 (segment (start 71.628 99.568) (end 60.96 88.9) (width 0.25) (layer B.Cu) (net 10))
 (segment (start 60.96 54.864) (end 61.976 53.848) (width 0.25) (layer B.Cu) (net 10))
 (segment (start 71.12 124.968) (end 74.93 124.968) (width 0.25) (layer B.Cu) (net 11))
 (segment (start 71.12 126.492) (end 71.12 124.968) (width 0.25) (layer B.Cu) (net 11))
 (segment (start 68.072 127.508) (end 70.104 127.508) (width 0.25) (layer B.Cu) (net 11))
 (segment (start 70.104 127.508) (end 71.12 126.492) (width 0.25) (layer B.Cu) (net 11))
 (segment (start 67.056 126.492) (end 68.072 127.508) (width 0.25) (layer B.Cu) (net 11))
 (segment (start 67.056 119.38) (end 67.056 126.492) (width 0.25) (layer B.Cu) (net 11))
 (segment (start 60.452 53.848) (end 60.452 112.776) (width 0.25) (layer B.Cu) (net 11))
 (segment (start 61.468 52.832) (end 60.452 53.848) (width 0.25) (layer B.Cu) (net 11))
 (segment (start 72.363949 52.832) (end 61.468 52.832) (width 0.25) (layer B.Cu) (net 11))
 (segment (start 60.452 112.776) (end 67.056 119.38) (width 0.25) (layer B.Cu) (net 11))
 (segment (start 77.47 57.938051) (end 72.363949 52.832) (width 0.25) (layer B.Cu) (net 11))
 (segment (start 77.47 58.928) (end 77.47 57.938051) (width 0.25) (layer B.Cu) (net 11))
 (segment (start 73.66 133.978) (end 73.66 132.588) (width 0.25) (layer B.Cu) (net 16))
 (segment (start 73.66 132.588) (end 80.264 125.984) (width 0.25) (layer B.Cu) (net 16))
 (segment (start 80.264 122.174) (end 82.55 119.888) (width 0.25) (layer B.Cu) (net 16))
 (segment (start 80.264 125.984) (end 80.264 122.174) (width 0.25) (layer B.Cu) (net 16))
 (segment (start 66.668 106.68) (end 64.77 108.578) (width 0.25) (layer F.Cu) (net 17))
 (segment (start 76.2 106.68) (end 66.668 106.68) (width 0.25) (layer F.Cu) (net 17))
 (segment (start 79.248 109.728) (end 76.2 106.68) (width 0.25) (layer F.Cu) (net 17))
 (segment (start 79.248 111.506) (end 79.248 109.728) (width 0.25) (layer F.Cu) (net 17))
 (segment (start 82.55 114.808) (end 79.248 111.506) (width 0.25) (layer F.Cu) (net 17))
 (segment (start 74.93 114.808) (end 71.628 114.808) (width 0.25) (layer B.Cu) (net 2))
 (segment (start 71.628 114.808) (end 69.596 112.776) (width 0.25) (layer B.Cu) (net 2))
 (segment (start 69.596 102.242) (end 66.16 98.806) (width 0.25) (layer B.Cu) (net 2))
 (segment (start 69.596 112.776) (end 69.596 102.242) (width 0.25) (layer B.Cu) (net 2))
 (segment (start 82.55 73.272) (end 80.906 71.628) (width 0.25) (layer B.Cu) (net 4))
 (segment (start 80.906 71.628) (end 78.232 71.628) (width 0.25) (layer B.Cu) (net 4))
 (segment (start 78.232 71.628) (end 75.692 74.168) (width 0.25) (layer B.Cu) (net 4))
 (segment (start 74.93 119.888) (end 76.708 118.11) (width 0.25) (layer B.Cu) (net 4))
 (segment (start 76.708 118.11) (end 76.708 108.204) (width 0.25) (layer B.Cu) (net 4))
 (segment (start 76.708 108.204) (end 75.692 107.188) (width 0.25) (layer B.Cu) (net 4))
 (segment (start 75.692 107.188) (end 75.692 89.916) (width 0.25) (layer B.Cu) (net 4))
 (segment (start 75.692 89.916) (end 75.692 90.424) (width 0.25) (layer B.Cu) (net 4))
 (segment (start 75.692 74.168) (end 75.692 89.916) (width 0.25) (layer B.Cu) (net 4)))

